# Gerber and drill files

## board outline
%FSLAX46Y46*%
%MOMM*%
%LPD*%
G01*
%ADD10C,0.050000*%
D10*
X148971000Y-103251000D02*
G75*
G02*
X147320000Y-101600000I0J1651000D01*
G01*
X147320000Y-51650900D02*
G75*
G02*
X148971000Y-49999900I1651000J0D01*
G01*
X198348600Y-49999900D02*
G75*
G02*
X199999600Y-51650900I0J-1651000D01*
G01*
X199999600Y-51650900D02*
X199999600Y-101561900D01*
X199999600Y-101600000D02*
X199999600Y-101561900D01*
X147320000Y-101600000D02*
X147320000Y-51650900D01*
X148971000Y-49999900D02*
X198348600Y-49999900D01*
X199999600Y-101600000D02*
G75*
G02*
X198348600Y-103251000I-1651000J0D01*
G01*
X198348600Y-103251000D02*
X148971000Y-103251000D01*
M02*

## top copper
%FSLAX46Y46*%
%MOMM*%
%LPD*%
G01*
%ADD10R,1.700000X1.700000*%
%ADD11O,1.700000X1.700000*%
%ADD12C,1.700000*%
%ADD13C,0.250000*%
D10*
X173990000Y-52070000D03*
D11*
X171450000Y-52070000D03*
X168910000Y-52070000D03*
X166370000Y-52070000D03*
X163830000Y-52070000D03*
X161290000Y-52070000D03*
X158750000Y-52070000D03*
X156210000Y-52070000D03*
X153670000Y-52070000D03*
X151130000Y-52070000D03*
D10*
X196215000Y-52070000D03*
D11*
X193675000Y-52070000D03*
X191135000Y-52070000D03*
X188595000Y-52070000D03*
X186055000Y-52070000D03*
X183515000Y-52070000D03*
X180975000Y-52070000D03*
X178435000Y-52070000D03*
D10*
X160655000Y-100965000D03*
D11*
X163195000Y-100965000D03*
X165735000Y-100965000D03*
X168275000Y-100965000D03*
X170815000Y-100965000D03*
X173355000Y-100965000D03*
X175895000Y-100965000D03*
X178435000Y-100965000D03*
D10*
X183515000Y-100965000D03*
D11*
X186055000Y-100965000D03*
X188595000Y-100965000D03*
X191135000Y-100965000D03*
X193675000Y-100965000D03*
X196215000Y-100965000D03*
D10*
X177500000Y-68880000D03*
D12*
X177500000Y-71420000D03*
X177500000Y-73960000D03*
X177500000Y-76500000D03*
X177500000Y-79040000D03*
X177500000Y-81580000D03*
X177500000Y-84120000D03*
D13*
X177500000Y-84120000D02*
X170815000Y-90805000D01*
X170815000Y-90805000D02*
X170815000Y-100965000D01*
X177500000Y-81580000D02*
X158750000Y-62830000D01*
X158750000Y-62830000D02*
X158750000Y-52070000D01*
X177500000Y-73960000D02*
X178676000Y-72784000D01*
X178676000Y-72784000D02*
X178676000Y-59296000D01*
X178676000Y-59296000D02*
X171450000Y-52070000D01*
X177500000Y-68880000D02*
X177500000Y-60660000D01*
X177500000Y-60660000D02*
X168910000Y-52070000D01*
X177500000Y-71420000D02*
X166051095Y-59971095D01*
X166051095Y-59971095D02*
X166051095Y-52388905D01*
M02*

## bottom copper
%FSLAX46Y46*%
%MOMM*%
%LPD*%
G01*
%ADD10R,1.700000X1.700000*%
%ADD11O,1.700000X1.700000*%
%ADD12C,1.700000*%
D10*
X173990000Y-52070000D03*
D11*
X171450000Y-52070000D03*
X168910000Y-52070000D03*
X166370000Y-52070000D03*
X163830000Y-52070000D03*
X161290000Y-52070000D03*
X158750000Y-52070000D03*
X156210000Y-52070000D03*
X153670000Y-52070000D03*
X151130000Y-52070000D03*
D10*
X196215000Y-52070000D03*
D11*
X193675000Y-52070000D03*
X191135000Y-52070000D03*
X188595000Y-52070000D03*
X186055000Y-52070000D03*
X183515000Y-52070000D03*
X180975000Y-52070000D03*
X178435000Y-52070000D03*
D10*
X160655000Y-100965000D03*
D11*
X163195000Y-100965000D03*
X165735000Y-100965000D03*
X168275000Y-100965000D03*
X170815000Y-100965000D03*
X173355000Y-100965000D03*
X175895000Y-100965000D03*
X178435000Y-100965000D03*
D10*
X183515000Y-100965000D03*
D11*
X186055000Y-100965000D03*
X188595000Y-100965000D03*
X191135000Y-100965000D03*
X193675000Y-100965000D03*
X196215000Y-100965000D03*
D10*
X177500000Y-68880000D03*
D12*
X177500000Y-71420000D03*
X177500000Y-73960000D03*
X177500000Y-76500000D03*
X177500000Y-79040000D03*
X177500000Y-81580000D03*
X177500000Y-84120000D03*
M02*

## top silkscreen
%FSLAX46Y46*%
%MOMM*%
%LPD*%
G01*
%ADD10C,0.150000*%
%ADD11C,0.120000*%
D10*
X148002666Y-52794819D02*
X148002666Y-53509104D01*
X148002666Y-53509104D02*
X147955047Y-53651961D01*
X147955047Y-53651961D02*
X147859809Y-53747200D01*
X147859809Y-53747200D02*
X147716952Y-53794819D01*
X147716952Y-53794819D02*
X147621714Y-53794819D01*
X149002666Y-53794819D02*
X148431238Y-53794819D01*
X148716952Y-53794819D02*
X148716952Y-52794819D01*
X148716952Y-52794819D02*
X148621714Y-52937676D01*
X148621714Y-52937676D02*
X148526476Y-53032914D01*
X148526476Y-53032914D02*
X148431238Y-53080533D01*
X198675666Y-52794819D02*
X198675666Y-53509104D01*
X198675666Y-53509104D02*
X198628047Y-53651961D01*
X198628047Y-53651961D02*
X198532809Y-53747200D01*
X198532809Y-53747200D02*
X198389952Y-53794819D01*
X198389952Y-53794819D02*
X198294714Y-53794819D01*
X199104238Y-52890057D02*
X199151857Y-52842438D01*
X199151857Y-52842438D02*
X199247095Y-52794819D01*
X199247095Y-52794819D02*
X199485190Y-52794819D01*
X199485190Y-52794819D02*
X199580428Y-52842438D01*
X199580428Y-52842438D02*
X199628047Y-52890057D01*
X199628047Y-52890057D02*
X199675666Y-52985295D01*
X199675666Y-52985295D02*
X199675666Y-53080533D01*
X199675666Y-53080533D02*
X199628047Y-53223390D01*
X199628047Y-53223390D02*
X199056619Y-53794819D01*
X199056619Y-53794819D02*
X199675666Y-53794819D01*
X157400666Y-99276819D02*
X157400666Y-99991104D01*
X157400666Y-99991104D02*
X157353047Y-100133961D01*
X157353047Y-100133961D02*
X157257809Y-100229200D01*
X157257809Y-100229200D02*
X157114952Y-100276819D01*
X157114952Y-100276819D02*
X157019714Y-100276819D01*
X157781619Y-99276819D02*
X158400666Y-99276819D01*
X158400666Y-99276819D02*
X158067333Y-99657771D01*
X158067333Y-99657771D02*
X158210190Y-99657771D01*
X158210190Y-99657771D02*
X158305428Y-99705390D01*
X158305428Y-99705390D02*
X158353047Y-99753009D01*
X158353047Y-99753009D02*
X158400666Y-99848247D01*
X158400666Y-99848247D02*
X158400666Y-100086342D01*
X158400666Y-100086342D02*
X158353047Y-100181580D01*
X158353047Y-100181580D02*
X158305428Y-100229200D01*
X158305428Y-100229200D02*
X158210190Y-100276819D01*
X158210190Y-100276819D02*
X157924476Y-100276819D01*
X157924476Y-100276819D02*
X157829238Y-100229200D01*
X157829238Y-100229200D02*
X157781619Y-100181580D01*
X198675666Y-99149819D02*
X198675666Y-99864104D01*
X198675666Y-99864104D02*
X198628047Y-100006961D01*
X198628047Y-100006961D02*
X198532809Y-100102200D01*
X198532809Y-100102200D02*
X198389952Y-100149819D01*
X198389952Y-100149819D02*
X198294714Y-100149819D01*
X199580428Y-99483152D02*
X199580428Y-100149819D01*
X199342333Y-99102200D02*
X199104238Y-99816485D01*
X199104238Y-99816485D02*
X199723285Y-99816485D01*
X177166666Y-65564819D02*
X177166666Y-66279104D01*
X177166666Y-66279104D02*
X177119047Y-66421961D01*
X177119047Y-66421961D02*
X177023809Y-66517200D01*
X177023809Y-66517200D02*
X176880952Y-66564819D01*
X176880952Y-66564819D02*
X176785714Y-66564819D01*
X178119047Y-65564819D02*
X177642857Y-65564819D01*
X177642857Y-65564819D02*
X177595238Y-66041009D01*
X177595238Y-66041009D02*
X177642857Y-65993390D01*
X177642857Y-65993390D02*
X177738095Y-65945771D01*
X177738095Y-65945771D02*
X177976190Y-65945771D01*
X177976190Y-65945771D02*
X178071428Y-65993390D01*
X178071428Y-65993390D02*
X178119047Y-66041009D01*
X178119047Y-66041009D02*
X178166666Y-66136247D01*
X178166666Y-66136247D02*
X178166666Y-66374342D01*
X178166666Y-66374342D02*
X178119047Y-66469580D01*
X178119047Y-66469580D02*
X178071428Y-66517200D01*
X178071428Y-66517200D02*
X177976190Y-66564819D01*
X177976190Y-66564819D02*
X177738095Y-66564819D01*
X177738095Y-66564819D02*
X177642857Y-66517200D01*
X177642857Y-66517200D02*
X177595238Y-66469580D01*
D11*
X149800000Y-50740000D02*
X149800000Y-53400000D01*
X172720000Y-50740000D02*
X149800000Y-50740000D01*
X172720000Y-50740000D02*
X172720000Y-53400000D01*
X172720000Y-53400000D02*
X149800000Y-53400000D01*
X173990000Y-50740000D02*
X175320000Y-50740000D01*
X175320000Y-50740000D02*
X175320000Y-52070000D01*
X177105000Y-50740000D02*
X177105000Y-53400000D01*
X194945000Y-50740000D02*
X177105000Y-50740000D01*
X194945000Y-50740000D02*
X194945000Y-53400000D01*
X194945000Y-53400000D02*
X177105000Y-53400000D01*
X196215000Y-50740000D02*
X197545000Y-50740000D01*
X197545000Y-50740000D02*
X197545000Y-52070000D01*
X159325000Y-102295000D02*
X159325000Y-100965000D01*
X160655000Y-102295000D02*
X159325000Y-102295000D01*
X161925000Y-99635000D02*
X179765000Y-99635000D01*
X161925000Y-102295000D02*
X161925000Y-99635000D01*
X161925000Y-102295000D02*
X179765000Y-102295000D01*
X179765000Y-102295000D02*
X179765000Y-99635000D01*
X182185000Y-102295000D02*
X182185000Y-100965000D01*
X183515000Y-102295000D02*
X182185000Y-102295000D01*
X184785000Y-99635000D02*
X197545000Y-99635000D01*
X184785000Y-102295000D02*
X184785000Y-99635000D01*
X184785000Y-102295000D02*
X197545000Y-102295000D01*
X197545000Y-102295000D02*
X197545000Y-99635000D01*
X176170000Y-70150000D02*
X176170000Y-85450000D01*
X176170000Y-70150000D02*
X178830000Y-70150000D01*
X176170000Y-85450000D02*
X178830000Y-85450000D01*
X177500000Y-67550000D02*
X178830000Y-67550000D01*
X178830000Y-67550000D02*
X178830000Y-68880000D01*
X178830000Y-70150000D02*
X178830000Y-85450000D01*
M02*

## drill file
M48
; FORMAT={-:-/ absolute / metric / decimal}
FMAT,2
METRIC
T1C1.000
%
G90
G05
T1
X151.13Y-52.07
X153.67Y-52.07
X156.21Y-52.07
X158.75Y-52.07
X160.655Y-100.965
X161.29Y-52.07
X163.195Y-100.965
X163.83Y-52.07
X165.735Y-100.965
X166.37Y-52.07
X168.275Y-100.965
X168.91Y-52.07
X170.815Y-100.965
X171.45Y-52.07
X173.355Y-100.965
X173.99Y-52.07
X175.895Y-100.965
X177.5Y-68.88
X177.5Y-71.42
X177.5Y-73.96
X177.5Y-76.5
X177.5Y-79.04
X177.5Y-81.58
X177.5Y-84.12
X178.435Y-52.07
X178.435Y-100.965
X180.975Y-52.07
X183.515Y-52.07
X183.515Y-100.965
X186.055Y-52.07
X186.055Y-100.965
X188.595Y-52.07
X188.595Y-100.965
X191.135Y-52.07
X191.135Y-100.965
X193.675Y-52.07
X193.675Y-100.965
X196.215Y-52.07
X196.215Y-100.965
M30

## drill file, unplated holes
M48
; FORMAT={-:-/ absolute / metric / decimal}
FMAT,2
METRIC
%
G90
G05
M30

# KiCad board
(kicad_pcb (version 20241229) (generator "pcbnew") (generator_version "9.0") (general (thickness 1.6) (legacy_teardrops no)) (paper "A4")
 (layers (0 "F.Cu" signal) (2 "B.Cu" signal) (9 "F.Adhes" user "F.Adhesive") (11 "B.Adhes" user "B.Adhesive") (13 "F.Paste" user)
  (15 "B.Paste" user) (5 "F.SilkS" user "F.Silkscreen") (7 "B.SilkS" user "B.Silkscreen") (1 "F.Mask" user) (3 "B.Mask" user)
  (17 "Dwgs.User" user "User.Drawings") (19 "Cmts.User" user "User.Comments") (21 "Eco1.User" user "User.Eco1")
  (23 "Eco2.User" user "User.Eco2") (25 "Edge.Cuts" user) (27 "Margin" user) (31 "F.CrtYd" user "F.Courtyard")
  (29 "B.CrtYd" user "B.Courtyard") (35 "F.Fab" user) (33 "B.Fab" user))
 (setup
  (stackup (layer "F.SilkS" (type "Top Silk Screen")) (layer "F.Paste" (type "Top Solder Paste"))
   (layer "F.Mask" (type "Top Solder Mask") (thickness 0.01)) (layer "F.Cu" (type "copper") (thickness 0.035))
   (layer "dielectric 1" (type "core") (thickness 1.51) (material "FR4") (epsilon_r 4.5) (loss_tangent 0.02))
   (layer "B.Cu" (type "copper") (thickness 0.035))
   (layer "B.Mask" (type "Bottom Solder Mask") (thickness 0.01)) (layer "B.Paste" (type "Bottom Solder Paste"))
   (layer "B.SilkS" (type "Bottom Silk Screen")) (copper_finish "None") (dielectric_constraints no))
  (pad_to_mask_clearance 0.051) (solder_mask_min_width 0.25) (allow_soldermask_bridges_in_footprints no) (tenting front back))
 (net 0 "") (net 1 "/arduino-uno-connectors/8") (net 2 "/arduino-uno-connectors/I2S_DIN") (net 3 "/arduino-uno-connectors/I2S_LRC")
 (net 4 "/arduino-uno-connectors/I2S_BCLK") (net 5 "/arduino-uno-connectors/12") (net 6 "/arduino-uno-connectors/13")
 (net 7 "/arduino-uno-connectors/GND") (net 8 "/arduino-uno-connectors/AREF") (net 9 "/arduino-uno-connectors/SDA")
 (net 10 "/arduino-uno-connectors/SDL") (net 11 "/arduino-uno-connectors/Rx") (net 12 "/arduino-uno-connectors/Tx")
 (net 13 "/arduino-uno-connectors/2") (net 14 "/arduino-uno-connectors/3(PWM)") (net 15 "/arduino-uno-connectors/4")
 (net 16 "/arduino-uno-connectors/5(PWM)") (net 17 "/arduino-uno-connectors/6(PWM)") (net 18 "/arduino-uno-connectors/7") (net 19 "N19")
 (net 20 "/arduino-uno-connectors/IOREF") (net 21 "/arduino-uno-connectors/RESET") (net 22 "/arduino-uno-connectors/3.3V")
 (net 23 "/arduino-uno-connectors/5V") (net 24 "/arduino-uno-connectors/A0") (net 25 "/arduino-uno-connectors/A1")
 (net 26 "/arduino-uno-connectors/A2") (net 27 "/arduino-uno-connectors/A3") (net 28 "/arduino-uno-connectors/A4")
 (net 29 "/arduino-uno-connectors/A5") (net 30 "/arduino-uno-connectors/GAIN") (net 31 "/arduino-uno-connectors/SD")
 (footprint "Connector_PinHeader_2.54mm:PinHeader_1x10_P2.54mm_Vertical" (layer "F.Cu") (at 173.99 52.07 -90)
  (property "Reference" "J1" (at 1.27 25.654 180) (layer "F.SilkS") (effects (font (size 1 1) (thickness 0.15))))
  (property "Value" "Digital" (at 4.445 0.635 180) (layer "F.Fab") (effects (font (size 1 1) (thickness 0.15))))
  (fp_line (start -1.33 24.19) (end 1.33 24.19) (stroke (width 0.12) (type solid)) (layer "F.SilkS"))
  (fp_line (start -1.33 1.27) (end -1.33 24.19) (stroke (width 0.12) (type solid)) (layer "F.SilkS"))
  (fp_line (start -1.33 1.27) (end 1.33 1.27) (stroke (width 0.12) (type solid)) (layer "F.SilkS"))
  (fp_line (start 1.33 1.27) (end 1.33 24.19) (stroke (width 0.12) (type solid)) (layer "F.SilkS"))
  (fp_line (start -1.33 0) (end -1.33 -1.33) (stroke (width 0.12) (type solid)) (layer "F.SilkS"))
  (fp_line (start -1.33 -1.33) (end 0 -1.33) (stroke (width 0.12) (type solid)) (layer "F.SilkS"))
  (pad "1" thru_hole rect (at 0 0 270) (size 1.7 1.7) (drill 1) (layers "*.Cu" "*.Mask") (remove_unused_layers no)
   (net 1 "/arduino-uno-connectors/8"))
  (pad "2" thru_hole oval (at 0 2.54 270) (size 1.7 1.7) (drill 1) (layers "*.Cu" "*.Mask") (remove_unused_layers no)
   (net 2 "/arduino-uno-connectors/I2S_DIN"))
  (pad "3" thru_hole oval (at 0 5.08 270) (size 1.7 1.7) (drill 1) (layers "*.Cu" "*.Mask") (remove_unused_layers no)
   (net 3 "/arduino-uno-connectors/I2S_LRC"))
  (pad "4" thru_hole oval (at 0 7.62 270) (size 1.7 1.7) (drill 1) (layers "*.Cu" "*.Mask") (remove_unused_layers no)
   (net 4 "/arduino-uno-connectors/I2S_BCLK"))
  (pad "5" thru_hole oval (at 0 10.16 270) (size 1.7 1.7) (drill 1) (layers "*.Cu" "*.Mask") (remove_unused_layers no)
   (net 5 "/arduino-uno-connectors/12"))
  (pad "6" thru_hole oval (at 0 12.7 270) (size 1.7 1.7) (drill 1) (layers "*.Cu" "*.Mask") (remove_unused_layers no)
   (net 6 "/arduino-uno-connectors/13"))
  (pad "7" thru_hole oval (at 0 15.24 270) (size 1.7 1.7) (drill 1) (layers "*.Cu" "*.Mask") (remove_unused_layers no)
   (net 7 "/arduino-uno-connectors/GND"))
  (pad "8" thru_hole oval (at 0 17.78 270) (size 1.7 1.7) (drill 1) (layers "*.Cu" "*.Mask") (remove_unused_layers no)
   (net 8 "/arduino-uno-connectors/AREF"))
  (pad "9" thru_hole oval (at 0 20.32 270) (size 1.7 1.7) (drill 1) (layers "*.Cu" "*.Mask") (remove_unused_layers no)
   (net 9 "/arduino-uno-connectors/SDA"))
  (pad "10" thru_hole oval (at 0 22.86 270) (size 1.7 1.7) (drill 1) (layers "*.Cu" "*.Mask") (remove_unused_layers no)
   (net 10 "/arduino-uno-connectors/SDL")))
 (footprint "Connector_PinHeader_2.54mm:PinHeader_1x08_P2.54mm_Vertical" (layer "F.Cu") (at 196.215 52.07 -90)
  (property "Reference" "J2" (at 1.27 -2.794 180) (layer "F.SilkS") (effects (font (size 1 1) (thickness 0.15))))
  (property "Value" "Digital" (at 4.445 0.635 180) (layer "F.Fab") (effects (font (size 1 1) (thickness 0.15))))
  (fp_line (start -1.33 19.11) (end 1.33 19.11) (stroke (width 0.12) (type solid)) (layer "F.SilkS"))
  (fp_line (start -1.33 1.27) (end -1.33 19.11) (stroke (width 0.12) (type solid)) (layer "F.SilkS"))
  (fp_line (start -1.33 1.27) (end 1.33 1.27) (stroke (width 0.12) (type solid)) (layer "F.SilkS"))
  (fp_line (start 1.33 1.27) (end 1.33 19.11) (stroke (width 0.12) (type solid)) (layer "F.SilkS"))
  (fp_line (start -1.33 0) (end -1.33 -1.33) (stroke (width 0.12) (type solid)) (layer "F.SilkS"))
  (fp_line (start -1.33 -1.33) (end 0 -1.33) (stroke (width 0.12) (type solid)) (layer "F.SilkS"))
  (pad "1" thru_hole rect (at 0 0 270) (size 1.7 1.7) (drill 1) (layers "*.Cu" "*.Mask") (remove_unused_layers no)
   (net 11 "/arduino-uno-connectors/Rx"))
  (pad "2" thru_hole oval (at 0 2.54 270) (size 1.7 1.7) (drill 1) (layers "*.Cu" "*.Mask") (remove_unused_layers no)
   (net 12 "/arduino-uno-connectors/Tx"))
  (pad "3" thru_hole oval (at 0 5.08 270) (size 1.7 1.7) (drill 1) (layers "*.Cu" "*.Mask") (remove_unused_layers no)
   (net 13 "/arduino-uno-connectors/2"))
  (pad "4" thru_hole oval (at 0 7.62 270) (size 1.7 1.7) (drill 1) (layers "*.Cu" "*.Mask") (remove_unused_layers no)
   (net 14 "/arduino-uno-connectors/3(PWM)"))
  (pad "5" thru_hole oval (at 0 10.16 270) (size 1.7 1.7) (drill 1) (layers "*.Cu" "*.Mask") (remove_unused_layers no)
   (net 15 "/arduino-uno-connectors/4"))
  (pad "6" thru_hole oval (at 0 12.7 270) (size 1.7 1.7) (drill 1) (layers "*.Cu" "*.Mask") (remove_unused_layers no)
   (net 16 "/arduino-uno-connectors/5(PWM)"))
  (pad "7" thru_hole oval (at 0 15.24 270) (size 1.7 1.7) (drill 1) (layers "*.Cu" "*.Mask") (remove_unused_layers no)
   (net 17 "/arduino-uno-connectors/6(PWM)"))
  (pad "8" thru_hole oval (at 0 17.78 270) (size 1.7 1.7) (drill 1) (layers "*.Cu" "*.Mask") (remove_unused_layers no)
   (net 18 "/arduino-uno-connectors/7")))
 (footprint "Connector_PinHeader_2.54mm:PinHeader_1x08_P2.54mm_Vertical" (layer "F.Cu") (at 160.655 100.965 90)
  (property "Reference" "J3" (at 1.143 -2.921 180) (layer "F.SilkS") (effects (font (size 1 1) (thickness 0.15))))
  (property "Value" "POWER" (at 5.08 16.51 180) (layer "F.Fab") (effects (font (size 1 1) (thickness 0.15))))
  (fp_line (start -1.33 -1.33) (end 0 -1.33) (stroke (width 0.12) (type solid)) (layer "F.SilkS"))
  (fp_line (start -1.33 0) (end -1.33 -1.33) (stroke (width 0.12) (type solid)) (layer "F.SilkS"))
  (fp_line (start 1.33 1.27) (end 1.33 19.11) (stroke (width 0.12) (type solid)) (layer "F.SilkS"))
  (fp_line (start -1.33 1.27) (end 1.33 1.27) (stroke (width 0.12) (type solid)) (layer "F.SilkS"))
  (fp_line (start -1.33 1.27) (end -1.33 19.11) (stroke (width 0.12) (type solid)) (layer "F.SilkS"))
  (fp_line (start -1.33 19.11) (end 1.33 19.11) (stroke (width 0.12) (type solid)) (layer "F.SilkS"))
  (pad "1" thru_hole rect (at 0 0 90) (size 1.7 1.7) (drill 1) (layers "*.Cu" "*.Mask") (remove_unused_layers no) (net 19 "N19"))
  (pad "2" thru_hole oval (at 0 2.54 90) (size 1.7 1.7) (drill 1) (layers "*.Cu" "*.Mask") (remove_unused_layers no)
   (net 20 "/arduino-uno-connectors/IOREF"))
  (pad "3" thru_hole oval (at 0 5.08 90) (size 1.7 1.7) (drill 1) (layers "*.Cu" "*.Mask") (remove_unused_layers no)
   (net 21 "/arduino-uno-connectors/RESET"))
  (pad "4" thru_hole oval (at 0 7.62 90) (size 1.7 1.7) (drill 1) (layers "*.Cu" "*.Mask") (remove_unused_layers no)
   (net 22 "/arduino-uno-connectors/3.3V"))
  (pad "5" thru_hole oval (at 0 10.16 90) (size 1.7 1.7) (drill 1) (layers "*.Cu" "*.Mask") (remove_unused_layers no)
   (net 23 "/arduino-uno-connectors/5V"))
  (pad "6" thru_hole oval (at 0 12.7 90) (size 1.7 1.7) (drill 1) (layers "*.Cu" "*.Mask") (remove_unused_layers no)
   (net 7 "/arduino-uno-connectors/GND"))
  (pad "7" thru_hole oval (at 0 15.24 90) (size 1.7 1.7) (drill 1) (layers "*.Cu" "*.Mask") (remove_unused_layers no)
   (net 7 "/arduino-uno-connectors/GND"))
  (pad "8" thru_hole oval (at 0 17.78 90) (size 1.7 1.7) (drill 1) (layers "*.Cu" "*.Mask") (remove_unused_layers no)
   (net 23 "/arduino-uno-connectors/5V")))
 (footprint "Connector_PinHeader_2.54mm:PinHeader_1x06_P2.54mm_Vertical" (layer "F.Cu") (at 183.515 100.965 90)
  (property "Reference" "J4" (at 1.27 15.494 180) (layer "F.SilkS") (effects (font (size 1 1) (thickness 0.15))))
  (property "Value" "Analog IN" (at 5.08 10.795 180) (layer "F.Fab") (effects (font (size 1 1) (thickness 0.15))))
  (fp_line (start -1.33 -1.33) (end 0 -1.33) (stroke (width 0.12) (type solid)) (layer "F.SilkS"))
  (fp_line (start -1.33 0) (end -1.33 -1.33) (stroke (width 0.12) (type solid)) (layer "F.SilkS"))
  (fp_line (start 1.33 1.27) (end 1.33 14.03) (stroke (width 0.12) (type solid)) (layer "F.SilkS"))
  (fp_line (start -1.33 1.27) (end 1.33 1.27) (stroke (width 0.12) (type solid)) (layer "F.SilkS"))
  (fp_line (start -1.33 1.27) (end -1.33 14.03) (stroke (width 0.12) (type solid)) (layer "F.SilkS"))
  (fp_line (start -1.33 14.03) (end 1.33 14.03) (stroke (width 0.12) (type solid)) (layer "F.SilkS"))
  (pad "1" thru_hole rect (at 0 0 90) (size 1.7 1.7) (drill 1) (layers "*.Cu" "*.Mask") (remove_unused_layers no)
   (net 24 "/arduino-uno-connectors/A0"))
  (pad "2" thru_hole oval (at 0 2.54 90) (size 1.7 1.7) (drill 1) (layers "*.Cu" "*.Mask") (remove_unused_layers no)
   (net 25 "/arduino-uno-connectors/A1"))
  (pad "3" thru_hole oval (at 0 5.08 90) (size 1.7 1.7) (drill 1) (layers "*.Cu" "*.Mask") (remove_unused_layers no)
   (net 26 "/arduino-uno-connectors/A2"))
  (pad "4" thru_hole oval (at 0 7.62 90) (size 1.7 1.7) (drill 1) (layers "*.Cu" "*.Mask") (remove_unused_layers no)
   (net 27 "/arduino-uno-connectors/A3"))
  (pad "5" thru_hole oval (at 0 10.16 90) (size 1.7 1.7) (drill 1) (layers "*.Cu" "*.Mask") (remove_unused_layers no)
   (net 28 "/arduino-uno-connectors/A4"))
  (pad "6" thru_hole oval (at 0 12.7 90) (size 1.7 1.7) (drill 1) (layers "*.Cu" "*.Mask") (remove_unused_layers no)
   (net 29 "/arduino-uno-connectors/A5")))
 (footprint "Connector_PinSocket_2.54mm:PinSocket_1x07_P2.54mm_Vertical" (layer "F.Cu") (at 177.5 68.88)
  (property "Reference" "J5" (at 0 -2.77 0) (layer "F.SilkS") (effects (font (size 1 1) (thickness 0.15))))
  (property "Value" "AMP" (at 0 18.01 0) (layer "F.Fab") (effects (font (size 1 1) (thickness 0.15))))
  (fp_line (start -1.33 1.27) (end -1.33 16.57) (stroke (width 0.12) (type solid)) (layer "F.SilkS"))
  (fp_line (start -1.33 1.27) (end 1.33 1.27) (stroke (width 0.12) (type solid)) (layer "F.SilkS"))
  (fp_line (start -1.33 16.57) (end 1.33 16.57) (stroke (width 0.12) (type solid)) (layer "F.SilkS"))
  (fp_line (start 0 -1.33) (end 1.33 -1.33) (stroke (width 0.12) (type solid)) (layer "F.SilkS"))
  (fp_line (start 1.33 -1.33) (end 1.33 0) (stroke (width 0.12) (type solid)) (layer "F.SilkS"))
  (fp_line (start 1.33 1.27) (end 1.33 16.57) (stroke (width 0.12) (type solid)) (layer "F.SilkS"))
  (pad "1" thru_hole rect (at 0 0) (size 1.7 1.7) (drill 1) (layers "*.Cu" "*.Mask") (remove_unused_layers no)
   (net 3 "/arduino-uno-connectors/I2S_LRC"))
  (pad "2" thru_hole circle (at 0 2.54) (size 1.7 1.7) (drill 1) (layers "*.Cu" "*.Mask") (remove_unused_layers no)
   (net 4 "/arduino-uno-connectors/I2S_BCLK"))
  (pad "3" thru_hole circle (at 0 5.08) (size 1.7 1.7) (drill 1) (layers "*.Cu" "*.Mask") (remove_unused_layers no)
   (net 2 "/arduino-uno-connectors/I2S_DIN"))
  (pad "4" thru_hole circle (at 0 7.62) (size 1.7 1.7) (drill 1) (layers "*.Cu" "*.Mask") (remove_unused_layers no)
   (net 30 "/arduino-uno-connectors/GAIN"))
  (pad "5" thru_hole circle (at 0 10.16) (size 1.7 1.7) (drill 1) (layers "*.Cu" "*.Mask") (remove_unused_layers no)
   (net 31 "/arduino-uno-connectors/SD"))
  (pad "6" thru_hole circle (at 0 12.7) (size 1.7 1.7) (drill 1) (layers "*.Cu" "*.Mask") (remove_unused_layers no)
   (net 7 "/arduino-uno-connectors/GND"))
  (pad "7" thru_hole circle (at 0 15.24) (size 1.7 1.7) (drill 1) (layers "*.Cu" "*.Mask") (remove_unused_layers no)
   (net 23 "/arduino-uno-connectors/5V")))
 (gr_arc (start 148.971 103.251) (mid 147.803567 102.767433) (end 147.32 101.6) (stroke (width 0.05) (type solid)) (layer "Edge.Cuts"))
 (gr_arc (start 147.32 51.6509) (mid 147.803567 50.483467) (end 148.971 49.9999) (stroke (width 0.05) (type solid)) (layer "Edge.Cuts"))
 (gr_arc (start 198.3486 49.9999) (mid 199.516033 50.483467) (end 199.9996 51.6509) (stroke (width 0.05) (type solid)) (layer "Edge.Cuts"))
 (gr_line (start 199.9996 51.6509) (end 199.9996 101.5619) (stroke (width 0.05) (type solid)) (layer "Edge.Cuts"))
 (gr_line (start 199.9996 101.6) (end 199.9996 101.5619) (stroke (width 0.05) (type solid)) (layer "Edge.Cuts"))
 (gr_line (start 147.32 101.6) (end 147.32 51.6509) (stroke (width 0.05) (type solid)) (layer "Edge.Cuts"))
 (gr_line (start 148.971 49.9999) (end 198.3486 49.9999) (stroke (width 0.05) (type solid)) (layer "Edge.Cuts"))
 (gr_arc (start 199.9996 101.6) (mid 199.516033 102.767433) (end 198.3486 103.251) (stroke (width 0.05) (type solid)) (layer "Edge.Cuts"))
 (gr_line (start 198.3486 103.251) (end 148.971 103.251) (stroke (width 0.05) (type solid)) (layer "Edge.Cuts"))
 (segment (start 177.5 84.12) (end 170.815 90.805) (width 0.25) (layer "F.Cu") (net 23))
 (segment (start 170.815 90.805) (end 170.815 100.965) (width 0.25) (layer "F.Cu") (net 23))
 (segment (start 158.75 62.83) (end 158.75 52.07) (width 0.25) (layer "F.Cu") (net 7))
 (segment (start 177.5 81.58) (end 158.75 62.83) (width 0.25) (layer "F.Cu") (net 7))
 (segment (start 177.5 73.96) (end 178.676 72.784) (width 0.25) (layer "F.Cu") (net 2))
 (segment (start 178.676 59.296) (end 171.45 52.07) (width 0.25) (layer "F.Cu") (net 2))
 (segment (start 178.676 72.784) (end 178.676 59.296) (width 0.25) (layer "F.Cu") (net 2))
 (segment (start 177.5 60.66) (end 168.91 52.07) (width 0.25) (layer "F.Cu") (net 3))
 (segment (start 177.5 68.88) (end 177.5 60.66) (width 0.25) (layer "F.Cu") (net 3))
 (segment (start 177.5 71.42) (end 166.051095 59.971095) (width 0.25) (layer "F.Cu") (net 4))
 (segment (start 166.051095 59.971095) (end 166.051095 52.388905) (width 0.25) (layer "F.Cu") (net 4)))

